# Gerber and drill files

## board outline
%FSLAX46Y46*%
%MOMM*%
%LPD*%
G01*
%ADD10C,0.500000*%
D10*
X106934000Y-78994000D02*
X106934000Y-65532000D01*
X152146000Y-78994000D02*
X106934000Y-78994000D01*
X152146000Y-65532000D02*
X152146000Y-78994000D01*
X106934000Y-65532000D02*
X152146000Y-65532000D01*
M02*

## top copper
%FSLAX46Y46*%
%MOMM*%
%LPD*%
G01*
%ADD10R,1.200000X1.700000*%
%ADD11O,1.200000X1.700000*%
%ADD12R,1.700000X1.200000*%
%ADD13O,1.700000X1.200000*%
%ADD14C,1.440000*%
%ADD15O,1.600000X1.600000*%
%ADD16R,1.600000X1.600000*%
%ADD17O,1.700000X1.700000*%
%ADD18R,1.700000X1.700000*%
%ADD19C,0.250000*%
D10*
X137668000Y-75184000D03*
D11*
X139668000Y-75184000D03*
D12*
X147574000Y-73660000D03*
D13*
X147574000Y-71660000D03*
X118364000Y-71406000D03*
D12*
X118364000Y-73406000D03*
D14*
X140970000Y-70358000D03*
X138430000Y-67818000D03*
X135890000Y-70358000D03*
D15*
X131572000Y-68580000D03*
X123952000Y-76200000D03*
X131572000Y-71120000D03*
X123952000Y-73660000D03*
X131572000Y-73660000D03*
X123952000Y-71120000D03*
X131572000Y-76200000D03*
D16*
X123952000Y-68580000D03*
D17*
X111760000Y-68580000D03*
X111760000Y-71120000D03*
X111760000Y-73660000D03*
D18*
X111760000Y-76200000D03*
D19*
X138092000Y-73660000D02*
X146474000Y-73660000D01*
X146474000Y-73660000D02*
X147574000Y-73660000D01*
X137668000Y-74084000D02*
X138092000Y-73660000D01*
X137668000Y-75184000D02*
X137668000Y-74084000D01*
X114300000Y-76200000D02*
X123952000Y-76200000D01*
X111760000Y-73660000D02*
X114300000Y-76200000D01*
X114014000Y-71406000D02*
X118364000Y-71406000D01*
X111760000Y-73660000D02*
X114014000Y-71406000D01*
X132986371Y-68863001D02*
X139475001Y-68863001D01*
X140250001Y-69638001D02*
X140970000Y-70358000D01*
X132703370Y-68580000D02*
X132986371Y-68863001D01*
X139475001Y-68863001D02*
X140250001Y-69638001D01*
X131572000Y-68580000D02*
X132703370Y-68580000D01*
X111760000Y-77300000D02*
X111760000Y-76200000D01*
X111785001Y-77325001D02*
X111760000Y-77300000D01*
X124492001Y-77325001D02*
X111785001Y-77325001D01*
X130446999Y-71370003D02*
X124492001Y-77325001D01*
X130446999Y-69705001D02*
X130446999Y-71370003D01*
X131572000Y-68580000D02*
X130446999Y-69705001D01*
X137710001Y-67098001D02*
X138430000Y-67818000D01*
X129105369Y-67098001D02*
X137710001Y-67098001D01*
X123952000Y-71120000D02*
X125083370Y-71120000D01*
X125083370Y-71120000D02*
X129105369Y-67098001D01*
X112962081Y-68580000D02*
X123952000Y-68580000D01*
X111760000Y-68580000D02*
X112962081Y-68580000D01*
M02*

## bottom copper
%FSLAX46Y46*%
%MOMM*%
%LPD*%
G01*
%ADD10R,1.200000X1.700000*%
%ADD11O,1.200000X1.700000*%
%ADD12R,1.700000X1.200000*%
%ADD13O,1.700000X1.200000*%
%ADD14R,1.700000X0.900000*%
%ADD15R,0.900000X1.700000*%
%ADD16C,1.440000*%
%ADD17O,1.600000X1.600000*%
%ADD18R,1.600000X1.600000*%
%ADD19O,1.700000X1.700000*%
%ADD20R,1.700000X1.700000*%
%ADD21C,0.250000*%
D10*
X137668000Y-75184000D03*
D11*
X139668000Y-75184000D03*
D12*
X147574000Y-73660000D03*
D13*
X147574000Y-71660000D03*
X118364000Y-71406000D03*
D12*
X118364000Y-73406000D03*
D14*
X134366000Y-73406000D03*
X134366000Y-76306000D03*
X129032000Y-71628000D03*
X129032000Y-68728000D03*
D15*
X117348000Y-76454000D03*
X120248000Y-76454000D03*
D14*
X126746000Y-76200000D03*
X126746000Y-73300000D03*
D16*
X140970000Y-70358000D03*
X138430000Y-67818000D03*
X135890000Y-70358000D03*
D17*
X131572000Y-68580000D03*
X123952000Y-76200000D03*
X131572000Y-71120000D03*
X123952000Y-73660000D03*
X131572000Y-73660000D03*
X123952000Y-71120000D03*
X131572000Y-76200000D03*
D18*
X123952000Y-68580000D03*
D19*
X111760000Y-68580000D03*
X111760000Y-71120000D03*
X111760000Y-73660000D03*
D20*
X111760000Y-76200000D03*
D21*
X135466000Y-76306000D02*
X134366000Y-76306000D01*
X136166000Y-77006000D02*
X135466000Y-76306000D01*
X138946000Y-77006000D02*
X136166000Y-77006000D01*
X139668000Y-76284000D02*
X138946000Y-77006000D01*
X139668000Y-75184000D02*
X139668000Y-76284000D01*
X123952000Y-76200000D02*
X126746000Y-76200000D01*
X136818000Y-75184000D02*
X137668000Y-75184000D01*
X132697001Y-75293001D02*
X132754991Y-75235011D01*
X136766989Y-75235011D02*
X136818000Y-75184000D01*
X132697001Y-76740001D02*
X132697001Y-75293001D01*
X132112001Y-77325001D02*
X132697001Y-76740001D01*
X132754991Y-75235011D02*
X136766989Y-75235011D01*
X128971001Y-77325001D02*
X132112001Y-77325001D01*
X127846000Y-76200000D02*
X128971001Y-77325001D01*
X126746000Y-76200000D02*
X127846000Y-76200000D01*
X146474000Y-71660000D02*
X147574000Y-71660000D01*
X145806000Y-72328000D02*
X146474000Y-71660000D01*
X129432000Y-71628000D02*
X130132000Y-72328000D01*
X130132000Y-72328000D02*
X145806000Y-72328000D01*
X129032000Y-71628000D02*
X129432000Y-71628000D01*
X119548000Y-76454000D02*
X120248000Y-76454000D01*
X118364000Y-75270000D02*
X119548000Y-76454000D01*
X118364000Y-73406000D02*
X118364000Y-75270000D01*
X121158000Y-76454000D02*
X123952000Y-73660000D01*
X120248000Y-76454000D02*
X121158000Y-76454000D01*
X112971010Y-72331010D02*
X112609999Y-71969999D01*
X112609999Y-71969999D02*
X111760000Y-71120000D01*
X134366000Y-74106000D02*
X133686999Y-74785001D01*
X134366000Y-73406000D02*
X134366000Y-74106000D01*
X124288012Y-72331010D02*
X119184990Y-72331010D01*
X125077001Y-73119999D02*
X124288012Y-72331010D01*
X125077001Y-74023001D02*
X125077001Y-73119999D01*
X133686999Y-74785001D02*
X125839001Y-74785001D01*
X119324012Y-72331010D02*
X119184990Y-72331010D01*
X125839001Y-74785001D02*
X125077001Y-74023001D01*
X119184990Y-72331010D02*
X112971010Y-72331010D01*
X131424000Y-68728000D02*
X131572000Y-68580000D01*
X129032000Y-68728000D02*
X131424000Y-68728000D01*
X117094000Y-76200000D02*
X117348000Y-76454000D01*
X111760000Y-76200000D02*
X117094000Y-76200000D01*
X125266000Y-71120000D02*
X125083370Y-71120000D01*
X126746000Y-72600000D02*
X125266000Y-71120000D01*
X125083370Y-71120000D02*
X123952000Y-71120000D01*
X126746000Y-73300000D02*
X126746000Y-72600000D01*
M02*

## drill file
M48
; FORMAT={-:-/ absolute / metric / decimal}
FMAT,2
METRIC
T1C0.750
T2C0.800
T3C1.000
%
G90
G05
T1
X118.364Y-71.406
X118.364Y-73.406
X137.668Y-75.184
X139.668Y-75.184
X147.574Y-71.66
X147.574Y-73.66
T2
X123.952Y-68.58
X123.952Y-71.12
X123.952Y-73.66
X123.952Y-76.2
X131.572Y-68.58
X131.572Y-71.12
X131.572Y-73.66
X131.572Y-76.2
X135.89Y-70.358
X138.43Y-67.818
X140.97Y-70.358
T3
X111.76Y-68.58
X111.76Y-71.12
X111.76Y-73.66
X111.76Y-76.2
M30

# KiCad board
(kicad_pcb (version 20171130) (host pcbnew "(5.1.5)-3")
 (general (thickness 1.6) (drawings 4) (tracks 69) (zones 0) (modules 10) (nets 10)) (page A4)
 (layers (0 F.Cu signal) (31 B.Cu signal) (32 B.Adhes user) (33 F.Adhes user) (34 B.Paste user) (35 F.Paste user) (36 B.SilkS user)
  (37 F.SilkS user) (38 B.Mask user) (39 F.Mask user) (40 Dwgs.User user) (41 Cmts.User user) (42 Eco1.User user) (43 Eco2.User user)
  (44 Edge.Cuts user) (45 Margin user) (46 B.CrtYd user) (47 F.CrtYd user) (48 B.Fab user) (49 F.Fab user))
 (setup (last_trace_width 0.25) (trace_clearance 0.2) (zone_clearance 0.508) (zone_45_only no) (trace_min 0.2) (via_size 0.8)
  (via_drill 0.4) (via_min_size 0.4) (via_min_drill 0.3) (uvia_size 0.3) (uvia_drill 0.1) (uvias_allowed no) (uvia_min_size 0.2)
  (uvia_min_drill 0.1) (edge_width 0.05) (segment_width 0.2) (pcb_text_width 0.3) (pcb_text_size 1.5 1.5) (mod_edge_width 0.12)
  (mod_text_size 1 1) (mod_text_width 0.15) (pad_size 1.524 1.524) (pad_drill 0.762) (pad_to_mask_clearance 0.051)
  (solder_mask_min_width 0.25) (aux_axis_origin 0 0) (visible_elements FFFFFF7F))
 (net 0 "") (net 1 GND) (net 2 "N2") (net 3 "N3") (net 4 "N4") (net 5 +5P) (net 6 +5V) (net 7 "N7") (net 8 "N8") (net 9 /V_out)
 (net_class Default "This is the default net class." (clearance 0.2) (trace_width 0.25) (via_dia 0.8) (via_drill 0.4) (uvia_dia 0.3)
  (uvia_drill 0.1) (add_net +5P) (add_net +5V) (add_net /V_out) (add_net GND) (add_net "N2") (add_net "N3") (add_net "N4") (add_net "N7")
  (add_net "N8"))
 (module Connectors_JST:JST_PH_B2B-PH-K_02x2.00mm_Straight (layer F.Cu) (at 137.668 75.184)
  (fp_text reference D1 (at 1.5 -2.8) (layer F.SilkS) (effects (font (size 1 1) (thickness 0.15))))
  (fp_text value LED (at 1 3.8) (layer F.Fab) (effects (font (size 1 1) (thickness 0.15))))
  (pad 1 thru_hole rect (at 0 0) (size 1.2 1.7) (drill 0.75) (layers *.Cu *.Mask) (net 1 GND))
  (pad 2 thru_hole oval (at 2 0) (size 1.2 1.7) (drill 0.75) (layers *.Cu *.Mask) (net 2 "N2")))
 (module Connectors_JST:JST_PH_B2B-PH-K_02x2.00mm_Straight (layer F.Cu) (at 147.574 73.66 90)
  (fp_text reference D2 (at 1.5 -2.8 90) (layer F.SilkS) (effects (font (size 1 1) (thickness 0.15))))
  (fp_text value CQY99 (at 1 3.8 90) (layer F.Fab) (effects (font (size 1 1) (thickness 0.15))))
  (pad 1 thru_hole rect (at 0 0 90) (size 1.2 1.7) (drill 0.75) (layers *.Cu *.Mask) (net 1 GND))
  (pad 2 thru_hole oval (at 2 0 90) (size 1.2 1.7) (drill 0.75) (layers *.Cu *.Mask) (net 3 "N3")))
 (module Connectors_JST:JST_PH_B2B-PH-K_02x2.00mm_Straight (layer F.Cu) (at 118.364 73.406 90)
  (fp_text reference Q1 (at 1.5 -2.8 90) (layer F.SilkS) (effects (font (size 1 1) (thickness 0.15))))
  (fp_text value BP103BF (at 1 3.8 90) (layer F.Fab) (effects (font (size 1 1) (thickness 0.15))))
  (pad 2 thru_hole oval (at 2 0 90) (size 1.2 1.7) (drill 0.75) (layers *.Cu *.Mask) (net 1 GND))
  (pad 1 thru_hole rect (at 0 0 90) (size 1.2 1.7) (drill 0.75) (layers *.Cu *.Mask) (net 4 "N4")))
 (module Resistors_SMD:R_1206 (layer B.Cu) (at 134.366 74.856 270)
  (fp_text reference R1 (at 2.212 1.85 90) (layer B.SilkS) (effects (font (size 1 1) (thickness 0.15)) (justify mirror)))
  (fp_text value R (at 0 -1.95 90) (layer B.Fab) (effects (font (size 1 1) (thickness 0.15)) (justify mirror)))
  (pad 1 smd rect (at -1.45 0 270) (size 0.9 1.7) (layers B.Cu B.Paste B.Mask) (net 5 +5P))
  (pad 2 smd rect (at 1.45 0 270) (size 0.9 1.7) (layers B.Cu B.Paste B.Mask) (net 2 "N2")))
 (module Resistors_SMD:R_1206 (layer B.Cu) (at 129.032 70.178 270)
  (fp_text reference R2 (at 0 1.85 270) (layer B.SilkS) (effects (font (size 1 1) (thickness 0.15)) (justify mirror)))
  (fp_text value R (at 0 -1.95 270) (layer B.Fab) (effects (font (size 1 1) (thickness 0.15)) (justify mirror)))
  (pad 2 smd rect (at 1.45 0 270) (size 0.9 1.7) (layers B.Cu B.Paste B.Mask) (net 3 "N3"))
  (pad 1 smd rect (at -1.45 0 270) (size 0.9 1.7) (layers B.Cu B.Paste B.Mask) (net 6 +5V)))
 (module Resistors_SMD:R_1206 (layer B.Cu) (at 118.798 76.454)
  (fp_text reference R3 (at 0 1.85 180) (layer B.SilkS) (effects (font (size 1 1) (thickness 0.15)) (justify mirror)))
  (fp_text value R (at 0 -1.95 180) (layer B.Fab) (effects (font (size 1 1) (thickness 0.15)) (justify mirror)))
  (pad 1 smd rect (at -1.45 0) (size 0.9 1.7) (layers B.Cu B.Paste B.Mask) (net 6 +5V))
  (pad 2 smd rect (at 1.45 0) (size 0.9 1.7) (layers B.Cu B.Paste B.Mask) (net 4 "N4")))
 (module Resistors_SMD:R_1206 (layer B.Cu) (at 126.746 74.75 270)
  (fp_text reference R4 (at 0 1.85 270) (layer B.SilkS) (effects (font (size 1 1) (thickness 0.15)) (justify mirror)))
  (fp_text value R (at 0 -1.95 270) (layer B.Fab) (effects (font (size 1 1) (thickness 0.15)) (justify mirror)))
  (pad 2 smd rect (at 1.45 0 270) (size 0.9 1.7) (layers B.Cu B.Paste B.Mask) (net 1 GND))
  (pad 1 smd rect (at -1.45 0 270) (size 0.9 1.7) (layers B.Cu B.Paste B.Mask) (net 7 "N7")))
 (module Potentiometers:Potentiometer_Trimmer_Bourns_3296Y (layer F.Cu) (at 135.89 70.358 180)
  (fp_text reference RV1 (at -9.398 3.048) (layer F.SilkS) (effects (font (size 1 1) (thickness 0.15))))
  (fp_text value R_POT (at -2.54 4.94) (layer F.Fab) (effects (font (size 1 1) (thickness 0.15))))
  (pad 3 thru_hole circle (at -5.08 0 180) (size 1.44 1.44) (drill 0.8) (layers *.Cu *.Mask) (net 6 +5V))
  (pad 2 thru_hole circle (at -2.54 2.54 180) (size 1.44 1.44) (drill 0.8) (layers *.Cu *.Mask) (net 7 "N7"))
  (pad 1 thru_hole circle (at 0 0 180) (size 1.44 1.44) (drill 0.8) (layers *.Cu *.Mask) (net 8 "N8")))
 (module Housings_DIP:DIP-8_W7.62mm (layer F.Cu) (at 123.952 68.58)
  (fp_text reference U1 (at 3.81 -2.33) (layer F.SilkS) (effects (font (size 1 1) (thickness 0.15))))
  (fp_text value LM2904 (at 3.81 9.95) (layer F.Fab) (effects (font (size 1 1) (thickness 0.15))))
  (pad 8 thru_hole oval (at 7.62 0) (size 1.6 1.6) (drill 0.8) (layers *.Cu *.Mask) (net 6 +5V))
  (pad 4 thru_hole oval (at 0 7.62) (size 1.6 1.6) (drill 0.8) (layers *.Cu *.Mask) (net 1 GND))
  (pad 7 thru_hole oval (at 7.62 2.54) (size 1.6 1.6) (drill 0.8) (layers *.Cu *.Mask))
  (pad 3 thru_hole oval (at 0 5.08) (size 1.6 1.6) (drill 0.8) (layers *.Cu *.Mask) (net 4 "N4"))
  (pad 6 thru_hole oval (at 7.62 5.08) (size 1.6 1.6) (drill 0.8) (layers *.Cu *.Mask))
  (pad 2 thru_hole oval (at 0 2.54) (size 1.6 1.6) (drill 0.8) (layers *.Cu *.Mask) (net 7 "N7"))
  (pad 5 thru_hole oval (at 7.62 7.62) (size 1.6 1.6) (drill 0.8) (layers *.Cu *.Mask))
  (pad 1 thru_hole rect (at 0 0) (size 1.6 1.6) (drill 0.8) (layers *.Cu *.Mask) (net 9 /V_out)))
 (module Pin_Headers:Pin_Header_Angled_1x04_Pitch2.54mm (layer F.Cu) (at 111.76 76.2 180)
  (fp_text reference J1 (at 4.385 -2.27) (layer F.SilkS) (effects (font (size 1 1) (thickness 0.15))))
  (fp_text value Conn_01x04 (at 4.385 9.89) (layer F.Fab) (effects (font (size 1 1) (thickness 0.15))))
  (pad 4 thru_hole oval (at 0 7.62 180) (size 1.7 1.7) (drill 1) (layers *.Cu *.Mask) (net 9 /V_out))
  (pad 3 thru_hole oval (at 0 5.08 180) (size 1.7 1.7) (drill 1) (layers *.Cu *.Mask) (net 5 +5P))
  (pad 2 thru_hole oval (at 0 2.54 180) (size 1.7 1.7) (drill 1) (layers *.Cu *.Mask) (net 1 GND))
  (pad 1 thru_hole rect (at 0 0 180) (size 1.7 1.7) (drill 1) (layers *.Cu *.Mask) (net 6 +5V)))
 (gr_line (start 106.934 78.994) (end 106.934 65.532) (layer Edge.Cuts) (width 0.5))
 (gr_line (start 152.146 78.994) (end 106.934 78.994) (layer Edge.Cuts) (width 0.5))
 (gr_line (start 152.146 65.532) (end 152.146 78.994) (layer Edge.Cuts) (width 0.5))
 (gr_line (start 106.934 65.532) (end 152.146 65.532) (layer Edge.Cuts) (width 0.5))
 (segment (start 135.466 76.306) (end 134.366 76.306) (width 0.25) (layer B.Cu) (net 2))
 (segment (start 136.166 77.006) (end 135.466 76.306) (width 0.25) (layer B.Cu) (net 2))
 (segment (start 138.946 77.006) (end 136.166 77.006) (width 0.25) (layer B.Cu) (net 2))
 (segment (start 139.668 76.284) (end 138.946 77.006) (width 0.25) (layer B.Cu) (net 2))
 (segment (start 139.668 75.184) (end 139.668 76.284) (width 0.25) (layer B.Cu) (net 2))
 (segment (start 138.092 73.66) (end 146.474 73.66) (width 0.25) (layer F.Cu) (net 1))
 (segment (start 146.474 73.66) (end 147.574 73.66) (width 0.25) (layer F.Cu) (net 1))
 (segment (start 137.668 74.084) (end 138.092 73.66) (width 0.25) (layer F.Cu) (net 1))
 (segment (start 137.668 75.184) (end 137.668 74.084) (width 0.25) (layer F.Cu) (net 1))
 (segment (start 123.952 76.2) (end 126.746 76.2) (width 0.25) (layer B.Cu) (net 1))
 (segment (start 114.3 76.2) (end 123.952 76.2) (width 0.25) (layer F.Cu) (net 1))
 (segment (start 111.76 73.66) (end 114.3 76.2) (width 0.25) (layer F.Cu) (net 1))
 (segment (start 114.014 71.406) (end 118.364 71.406) (width 0.25) (layer F.Cu) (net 1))
 (segment (start 111.76 73.66) (end 114.014 71.406) (width 0.25) (layer F.Cu) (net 1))
 (segment (start 136.818 75.184) (end 137.668 75.184) (width 0.25) (layer B.Cu) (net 1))
 (segment (start 132.697001 75.293001) (end 132.754991 75.235011) (width 0.25) (layer B.Cu) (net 1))
 (segment (start 136.766989 75.235011) (end 136.818 75.184) (width 0.25) (layer B.Cu) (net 1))
 (segment (start 132.697001 76.740001) (end 132.697001 75.293001) (width 0.25) (layer B.Cu) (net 1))
 (segment (start 132.112001 77.325001) (end 132.697001 76.740001) (width 0.25) (layer B.Cu) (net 1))
 (segment (start 132.754991 75.235011) (end 136.766989 75.235011) (width 0.25) (layer B.Cu) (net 1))
 (segment (start 128.971001 77.325001) (end 132.112001 77.325001) (width 0.25) (layer B.Cu) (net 1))
 (segment (start 127.846 76.2) (end 128.971001 77.325001) (width 0.25) (layer B.Cu) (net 1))
 (segment (start 126.746 76.2) (end 127.846 76.2) (width 0.25) (layer B.Cu) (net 1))
 (segment (start 146.474 71.66) (end 147.574 71.66) (width 0.25) (layer B.Cu) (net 3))
 (segment (start 145.806 72.328) (end 146.474 71.66) (width 0.25) (layer B.Cu) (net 3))
 (segment (start 129.432 71.628) (end 130.132 72.328) (width 0.25) (layer B.Cu) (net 3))
 (segment (start 130.132 72.328) (end 145.806 72.328) (width 0.25) (layer B.Cu) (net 3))
 (segment (start 129.032 71.628) (end 129.432 71.628) (width 0.25) (layer B.Cu) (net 3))
 (segment (start 119.548 76.454) (end 120.248 76.454) (width 0.25) (layer B.Cu) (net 4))
 (segment (start 118.364 75.27) (end 119.548 76.454) (width 0.25) (layer B.Cu) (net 4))
 (segment (start 118.364 73.406) (end 118.364 75.27) (width 0.25) (layer B.Cu) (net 4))
 (segment (start 121.158 76.454) (end 123.952 73.66) (width 0.25) (layer B.Cu) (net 4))
 (segment (start 120.248 76.454) (end 121.158 76.454) (width 0.25) (layer B.Cu) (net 4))
 (segment (start 112.97101 72.33101) (end 112.609999 71.969999) (width 0.25) (layer B.Cu) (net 5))
 (segment (start 112.609999 71.969999) (end 111.76 71.12) (width 0.25) (layer B.Cu) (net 5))
 (segment (start 134.366 74.106) (end 133.686999 74.785001) (width 0.25) (layer B.Cu) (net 5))
 (segment (start 134.366 73.406) (end 134.366 74.106) (width 0.25) (layer B.Cu) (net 5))
 (segment (start 124.288012 72.33101) (end 119.18499 72.33101) (width 0.25) (layer B.Cu) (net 5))
 (segment (start 125.077001 73.119999) (end 124.288012 72.33101) (width 0.25) (layer B.Cu) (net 5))
 (segment (start 125.077001 74.023001) (end 125.077001 73.119999) (width 0.25) (layer B.Cu) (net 5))
 (segment (start 133.686999 74.785001) (end 125.839001 74.785001) (width 0.25) (layer B.Cu) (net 5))
 (segment (start 119.324012 72.33101) (end 119.18499 72.33101) (width 0.25) (layer B.Cu) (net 5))
 (segment (start 125.839001 74.785001) (end 125.077001 74.023001) (width 0.25) (layer B.Cu) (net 5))
 (segment (start 119.18499 72.33101) (end 112.97101 72.33101) (width 0.25) (layer B.Cu) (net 5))
 (segment (start 132.986371 68.863001) (end 139.475001 68.863001) (width 0.25) (layer F.Cu) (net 6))
 (segment (start 140.250001 69.638001) (end 140.97 70.358) (width 0.25) (layer F.Cu) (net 6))
 (segment (start 132.70337 68.58) (end 132.986371 68.863001) (width 0.25) (layer F.Cu) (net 6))
 (segment (start 139.475001 68.863001) (end 140.250001 69.638001) (width 0.25) (layer F.Cu) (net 6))
 (segment (start 131.572 68.58) (end 132.70337 68.58) (width 0.25) (layer F.Cu) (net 6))
 (segment (start 131.424 68.728) (end 131.572 68.58) (width 0.25) (layer B.Cu) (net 6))
 (segment (start 129.032 68.728) (end 131.424 68.728) (width 0.25) (layer B.Cu) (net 6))
 (segment (start 117.094 76.2) (end 117.348 76.454) (width 0.25) (layer B.Cu) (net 6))
 (segment (start 111.76 76.2) (end 117.094 76.2) (width 0.25) (layer B.Cu) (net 6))
 (segment (start 111.76 77.3) (end 111.76 76.2) (width 0.25) (layer F.Cu) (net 6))
 (segment (start 111.785001 77.325001) (end 111.76 77.3) (width 0.25) (layer F.Cu) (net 6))
 (segment (start 124.492001 77.325001) (end 111.785001 77.325001) (width 0.25) (layer F.Cu) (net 6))
 (segment (start 130.446999 71.370003) (end 124.492001 77.325001) (width 0.25) (layer F.Cu) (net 6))
 (segment (start 130.446999 69.705001) (end 130.446999 71.370003) (width 0.25) (layer F.Cu) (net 6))
 (segment (start 131.572 68.58) (end 130.446999 69.705001) (width 0.25) (layer F.Cu) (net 6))
 (segment (start 137.710001 67.098001) (end 138.43 67.818) (width 0.25) (layer F.Cu) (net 7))
 (segment (start 129.105369 67.098001) (end 137.710001 67.098001) (width 0.25) (layer F.Cu) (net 7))
 (segment (start 123.952 71.12) (end 125.08337 71.12) (width 0.25) (layer F.Cu) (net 7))
 (segment (start 125.08337 71.12) (end 129.105369 67.098001) (width 0.25) (layer F.Cu) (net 7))
 (segment (start 125.266 71.12) (end 125.08337 71.12) (width 0.25) (layer B.Cu) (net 7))
 (segment (start 126.746 72.6) (end 125.266 71.12) (width 0.25) (layer B.Cu) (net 7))
 (segment (start 125.08337 71.12) (end 123.952 71.12) (width 0.25) (layer B.Cu) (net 7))
 (segment (start 126.746 73.3) (end 126.746 72.6) (width 0.25) (layer B.Cu) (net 7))
 (segment (start 112.962081 68.58) (end 123.952 68.58) (width 0.25) (layer F.Cu) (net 9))
 (segment (start 111.76 68.58) (end 112.962081 68.58) (width 0.25) (layer F.Cu) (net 9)))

